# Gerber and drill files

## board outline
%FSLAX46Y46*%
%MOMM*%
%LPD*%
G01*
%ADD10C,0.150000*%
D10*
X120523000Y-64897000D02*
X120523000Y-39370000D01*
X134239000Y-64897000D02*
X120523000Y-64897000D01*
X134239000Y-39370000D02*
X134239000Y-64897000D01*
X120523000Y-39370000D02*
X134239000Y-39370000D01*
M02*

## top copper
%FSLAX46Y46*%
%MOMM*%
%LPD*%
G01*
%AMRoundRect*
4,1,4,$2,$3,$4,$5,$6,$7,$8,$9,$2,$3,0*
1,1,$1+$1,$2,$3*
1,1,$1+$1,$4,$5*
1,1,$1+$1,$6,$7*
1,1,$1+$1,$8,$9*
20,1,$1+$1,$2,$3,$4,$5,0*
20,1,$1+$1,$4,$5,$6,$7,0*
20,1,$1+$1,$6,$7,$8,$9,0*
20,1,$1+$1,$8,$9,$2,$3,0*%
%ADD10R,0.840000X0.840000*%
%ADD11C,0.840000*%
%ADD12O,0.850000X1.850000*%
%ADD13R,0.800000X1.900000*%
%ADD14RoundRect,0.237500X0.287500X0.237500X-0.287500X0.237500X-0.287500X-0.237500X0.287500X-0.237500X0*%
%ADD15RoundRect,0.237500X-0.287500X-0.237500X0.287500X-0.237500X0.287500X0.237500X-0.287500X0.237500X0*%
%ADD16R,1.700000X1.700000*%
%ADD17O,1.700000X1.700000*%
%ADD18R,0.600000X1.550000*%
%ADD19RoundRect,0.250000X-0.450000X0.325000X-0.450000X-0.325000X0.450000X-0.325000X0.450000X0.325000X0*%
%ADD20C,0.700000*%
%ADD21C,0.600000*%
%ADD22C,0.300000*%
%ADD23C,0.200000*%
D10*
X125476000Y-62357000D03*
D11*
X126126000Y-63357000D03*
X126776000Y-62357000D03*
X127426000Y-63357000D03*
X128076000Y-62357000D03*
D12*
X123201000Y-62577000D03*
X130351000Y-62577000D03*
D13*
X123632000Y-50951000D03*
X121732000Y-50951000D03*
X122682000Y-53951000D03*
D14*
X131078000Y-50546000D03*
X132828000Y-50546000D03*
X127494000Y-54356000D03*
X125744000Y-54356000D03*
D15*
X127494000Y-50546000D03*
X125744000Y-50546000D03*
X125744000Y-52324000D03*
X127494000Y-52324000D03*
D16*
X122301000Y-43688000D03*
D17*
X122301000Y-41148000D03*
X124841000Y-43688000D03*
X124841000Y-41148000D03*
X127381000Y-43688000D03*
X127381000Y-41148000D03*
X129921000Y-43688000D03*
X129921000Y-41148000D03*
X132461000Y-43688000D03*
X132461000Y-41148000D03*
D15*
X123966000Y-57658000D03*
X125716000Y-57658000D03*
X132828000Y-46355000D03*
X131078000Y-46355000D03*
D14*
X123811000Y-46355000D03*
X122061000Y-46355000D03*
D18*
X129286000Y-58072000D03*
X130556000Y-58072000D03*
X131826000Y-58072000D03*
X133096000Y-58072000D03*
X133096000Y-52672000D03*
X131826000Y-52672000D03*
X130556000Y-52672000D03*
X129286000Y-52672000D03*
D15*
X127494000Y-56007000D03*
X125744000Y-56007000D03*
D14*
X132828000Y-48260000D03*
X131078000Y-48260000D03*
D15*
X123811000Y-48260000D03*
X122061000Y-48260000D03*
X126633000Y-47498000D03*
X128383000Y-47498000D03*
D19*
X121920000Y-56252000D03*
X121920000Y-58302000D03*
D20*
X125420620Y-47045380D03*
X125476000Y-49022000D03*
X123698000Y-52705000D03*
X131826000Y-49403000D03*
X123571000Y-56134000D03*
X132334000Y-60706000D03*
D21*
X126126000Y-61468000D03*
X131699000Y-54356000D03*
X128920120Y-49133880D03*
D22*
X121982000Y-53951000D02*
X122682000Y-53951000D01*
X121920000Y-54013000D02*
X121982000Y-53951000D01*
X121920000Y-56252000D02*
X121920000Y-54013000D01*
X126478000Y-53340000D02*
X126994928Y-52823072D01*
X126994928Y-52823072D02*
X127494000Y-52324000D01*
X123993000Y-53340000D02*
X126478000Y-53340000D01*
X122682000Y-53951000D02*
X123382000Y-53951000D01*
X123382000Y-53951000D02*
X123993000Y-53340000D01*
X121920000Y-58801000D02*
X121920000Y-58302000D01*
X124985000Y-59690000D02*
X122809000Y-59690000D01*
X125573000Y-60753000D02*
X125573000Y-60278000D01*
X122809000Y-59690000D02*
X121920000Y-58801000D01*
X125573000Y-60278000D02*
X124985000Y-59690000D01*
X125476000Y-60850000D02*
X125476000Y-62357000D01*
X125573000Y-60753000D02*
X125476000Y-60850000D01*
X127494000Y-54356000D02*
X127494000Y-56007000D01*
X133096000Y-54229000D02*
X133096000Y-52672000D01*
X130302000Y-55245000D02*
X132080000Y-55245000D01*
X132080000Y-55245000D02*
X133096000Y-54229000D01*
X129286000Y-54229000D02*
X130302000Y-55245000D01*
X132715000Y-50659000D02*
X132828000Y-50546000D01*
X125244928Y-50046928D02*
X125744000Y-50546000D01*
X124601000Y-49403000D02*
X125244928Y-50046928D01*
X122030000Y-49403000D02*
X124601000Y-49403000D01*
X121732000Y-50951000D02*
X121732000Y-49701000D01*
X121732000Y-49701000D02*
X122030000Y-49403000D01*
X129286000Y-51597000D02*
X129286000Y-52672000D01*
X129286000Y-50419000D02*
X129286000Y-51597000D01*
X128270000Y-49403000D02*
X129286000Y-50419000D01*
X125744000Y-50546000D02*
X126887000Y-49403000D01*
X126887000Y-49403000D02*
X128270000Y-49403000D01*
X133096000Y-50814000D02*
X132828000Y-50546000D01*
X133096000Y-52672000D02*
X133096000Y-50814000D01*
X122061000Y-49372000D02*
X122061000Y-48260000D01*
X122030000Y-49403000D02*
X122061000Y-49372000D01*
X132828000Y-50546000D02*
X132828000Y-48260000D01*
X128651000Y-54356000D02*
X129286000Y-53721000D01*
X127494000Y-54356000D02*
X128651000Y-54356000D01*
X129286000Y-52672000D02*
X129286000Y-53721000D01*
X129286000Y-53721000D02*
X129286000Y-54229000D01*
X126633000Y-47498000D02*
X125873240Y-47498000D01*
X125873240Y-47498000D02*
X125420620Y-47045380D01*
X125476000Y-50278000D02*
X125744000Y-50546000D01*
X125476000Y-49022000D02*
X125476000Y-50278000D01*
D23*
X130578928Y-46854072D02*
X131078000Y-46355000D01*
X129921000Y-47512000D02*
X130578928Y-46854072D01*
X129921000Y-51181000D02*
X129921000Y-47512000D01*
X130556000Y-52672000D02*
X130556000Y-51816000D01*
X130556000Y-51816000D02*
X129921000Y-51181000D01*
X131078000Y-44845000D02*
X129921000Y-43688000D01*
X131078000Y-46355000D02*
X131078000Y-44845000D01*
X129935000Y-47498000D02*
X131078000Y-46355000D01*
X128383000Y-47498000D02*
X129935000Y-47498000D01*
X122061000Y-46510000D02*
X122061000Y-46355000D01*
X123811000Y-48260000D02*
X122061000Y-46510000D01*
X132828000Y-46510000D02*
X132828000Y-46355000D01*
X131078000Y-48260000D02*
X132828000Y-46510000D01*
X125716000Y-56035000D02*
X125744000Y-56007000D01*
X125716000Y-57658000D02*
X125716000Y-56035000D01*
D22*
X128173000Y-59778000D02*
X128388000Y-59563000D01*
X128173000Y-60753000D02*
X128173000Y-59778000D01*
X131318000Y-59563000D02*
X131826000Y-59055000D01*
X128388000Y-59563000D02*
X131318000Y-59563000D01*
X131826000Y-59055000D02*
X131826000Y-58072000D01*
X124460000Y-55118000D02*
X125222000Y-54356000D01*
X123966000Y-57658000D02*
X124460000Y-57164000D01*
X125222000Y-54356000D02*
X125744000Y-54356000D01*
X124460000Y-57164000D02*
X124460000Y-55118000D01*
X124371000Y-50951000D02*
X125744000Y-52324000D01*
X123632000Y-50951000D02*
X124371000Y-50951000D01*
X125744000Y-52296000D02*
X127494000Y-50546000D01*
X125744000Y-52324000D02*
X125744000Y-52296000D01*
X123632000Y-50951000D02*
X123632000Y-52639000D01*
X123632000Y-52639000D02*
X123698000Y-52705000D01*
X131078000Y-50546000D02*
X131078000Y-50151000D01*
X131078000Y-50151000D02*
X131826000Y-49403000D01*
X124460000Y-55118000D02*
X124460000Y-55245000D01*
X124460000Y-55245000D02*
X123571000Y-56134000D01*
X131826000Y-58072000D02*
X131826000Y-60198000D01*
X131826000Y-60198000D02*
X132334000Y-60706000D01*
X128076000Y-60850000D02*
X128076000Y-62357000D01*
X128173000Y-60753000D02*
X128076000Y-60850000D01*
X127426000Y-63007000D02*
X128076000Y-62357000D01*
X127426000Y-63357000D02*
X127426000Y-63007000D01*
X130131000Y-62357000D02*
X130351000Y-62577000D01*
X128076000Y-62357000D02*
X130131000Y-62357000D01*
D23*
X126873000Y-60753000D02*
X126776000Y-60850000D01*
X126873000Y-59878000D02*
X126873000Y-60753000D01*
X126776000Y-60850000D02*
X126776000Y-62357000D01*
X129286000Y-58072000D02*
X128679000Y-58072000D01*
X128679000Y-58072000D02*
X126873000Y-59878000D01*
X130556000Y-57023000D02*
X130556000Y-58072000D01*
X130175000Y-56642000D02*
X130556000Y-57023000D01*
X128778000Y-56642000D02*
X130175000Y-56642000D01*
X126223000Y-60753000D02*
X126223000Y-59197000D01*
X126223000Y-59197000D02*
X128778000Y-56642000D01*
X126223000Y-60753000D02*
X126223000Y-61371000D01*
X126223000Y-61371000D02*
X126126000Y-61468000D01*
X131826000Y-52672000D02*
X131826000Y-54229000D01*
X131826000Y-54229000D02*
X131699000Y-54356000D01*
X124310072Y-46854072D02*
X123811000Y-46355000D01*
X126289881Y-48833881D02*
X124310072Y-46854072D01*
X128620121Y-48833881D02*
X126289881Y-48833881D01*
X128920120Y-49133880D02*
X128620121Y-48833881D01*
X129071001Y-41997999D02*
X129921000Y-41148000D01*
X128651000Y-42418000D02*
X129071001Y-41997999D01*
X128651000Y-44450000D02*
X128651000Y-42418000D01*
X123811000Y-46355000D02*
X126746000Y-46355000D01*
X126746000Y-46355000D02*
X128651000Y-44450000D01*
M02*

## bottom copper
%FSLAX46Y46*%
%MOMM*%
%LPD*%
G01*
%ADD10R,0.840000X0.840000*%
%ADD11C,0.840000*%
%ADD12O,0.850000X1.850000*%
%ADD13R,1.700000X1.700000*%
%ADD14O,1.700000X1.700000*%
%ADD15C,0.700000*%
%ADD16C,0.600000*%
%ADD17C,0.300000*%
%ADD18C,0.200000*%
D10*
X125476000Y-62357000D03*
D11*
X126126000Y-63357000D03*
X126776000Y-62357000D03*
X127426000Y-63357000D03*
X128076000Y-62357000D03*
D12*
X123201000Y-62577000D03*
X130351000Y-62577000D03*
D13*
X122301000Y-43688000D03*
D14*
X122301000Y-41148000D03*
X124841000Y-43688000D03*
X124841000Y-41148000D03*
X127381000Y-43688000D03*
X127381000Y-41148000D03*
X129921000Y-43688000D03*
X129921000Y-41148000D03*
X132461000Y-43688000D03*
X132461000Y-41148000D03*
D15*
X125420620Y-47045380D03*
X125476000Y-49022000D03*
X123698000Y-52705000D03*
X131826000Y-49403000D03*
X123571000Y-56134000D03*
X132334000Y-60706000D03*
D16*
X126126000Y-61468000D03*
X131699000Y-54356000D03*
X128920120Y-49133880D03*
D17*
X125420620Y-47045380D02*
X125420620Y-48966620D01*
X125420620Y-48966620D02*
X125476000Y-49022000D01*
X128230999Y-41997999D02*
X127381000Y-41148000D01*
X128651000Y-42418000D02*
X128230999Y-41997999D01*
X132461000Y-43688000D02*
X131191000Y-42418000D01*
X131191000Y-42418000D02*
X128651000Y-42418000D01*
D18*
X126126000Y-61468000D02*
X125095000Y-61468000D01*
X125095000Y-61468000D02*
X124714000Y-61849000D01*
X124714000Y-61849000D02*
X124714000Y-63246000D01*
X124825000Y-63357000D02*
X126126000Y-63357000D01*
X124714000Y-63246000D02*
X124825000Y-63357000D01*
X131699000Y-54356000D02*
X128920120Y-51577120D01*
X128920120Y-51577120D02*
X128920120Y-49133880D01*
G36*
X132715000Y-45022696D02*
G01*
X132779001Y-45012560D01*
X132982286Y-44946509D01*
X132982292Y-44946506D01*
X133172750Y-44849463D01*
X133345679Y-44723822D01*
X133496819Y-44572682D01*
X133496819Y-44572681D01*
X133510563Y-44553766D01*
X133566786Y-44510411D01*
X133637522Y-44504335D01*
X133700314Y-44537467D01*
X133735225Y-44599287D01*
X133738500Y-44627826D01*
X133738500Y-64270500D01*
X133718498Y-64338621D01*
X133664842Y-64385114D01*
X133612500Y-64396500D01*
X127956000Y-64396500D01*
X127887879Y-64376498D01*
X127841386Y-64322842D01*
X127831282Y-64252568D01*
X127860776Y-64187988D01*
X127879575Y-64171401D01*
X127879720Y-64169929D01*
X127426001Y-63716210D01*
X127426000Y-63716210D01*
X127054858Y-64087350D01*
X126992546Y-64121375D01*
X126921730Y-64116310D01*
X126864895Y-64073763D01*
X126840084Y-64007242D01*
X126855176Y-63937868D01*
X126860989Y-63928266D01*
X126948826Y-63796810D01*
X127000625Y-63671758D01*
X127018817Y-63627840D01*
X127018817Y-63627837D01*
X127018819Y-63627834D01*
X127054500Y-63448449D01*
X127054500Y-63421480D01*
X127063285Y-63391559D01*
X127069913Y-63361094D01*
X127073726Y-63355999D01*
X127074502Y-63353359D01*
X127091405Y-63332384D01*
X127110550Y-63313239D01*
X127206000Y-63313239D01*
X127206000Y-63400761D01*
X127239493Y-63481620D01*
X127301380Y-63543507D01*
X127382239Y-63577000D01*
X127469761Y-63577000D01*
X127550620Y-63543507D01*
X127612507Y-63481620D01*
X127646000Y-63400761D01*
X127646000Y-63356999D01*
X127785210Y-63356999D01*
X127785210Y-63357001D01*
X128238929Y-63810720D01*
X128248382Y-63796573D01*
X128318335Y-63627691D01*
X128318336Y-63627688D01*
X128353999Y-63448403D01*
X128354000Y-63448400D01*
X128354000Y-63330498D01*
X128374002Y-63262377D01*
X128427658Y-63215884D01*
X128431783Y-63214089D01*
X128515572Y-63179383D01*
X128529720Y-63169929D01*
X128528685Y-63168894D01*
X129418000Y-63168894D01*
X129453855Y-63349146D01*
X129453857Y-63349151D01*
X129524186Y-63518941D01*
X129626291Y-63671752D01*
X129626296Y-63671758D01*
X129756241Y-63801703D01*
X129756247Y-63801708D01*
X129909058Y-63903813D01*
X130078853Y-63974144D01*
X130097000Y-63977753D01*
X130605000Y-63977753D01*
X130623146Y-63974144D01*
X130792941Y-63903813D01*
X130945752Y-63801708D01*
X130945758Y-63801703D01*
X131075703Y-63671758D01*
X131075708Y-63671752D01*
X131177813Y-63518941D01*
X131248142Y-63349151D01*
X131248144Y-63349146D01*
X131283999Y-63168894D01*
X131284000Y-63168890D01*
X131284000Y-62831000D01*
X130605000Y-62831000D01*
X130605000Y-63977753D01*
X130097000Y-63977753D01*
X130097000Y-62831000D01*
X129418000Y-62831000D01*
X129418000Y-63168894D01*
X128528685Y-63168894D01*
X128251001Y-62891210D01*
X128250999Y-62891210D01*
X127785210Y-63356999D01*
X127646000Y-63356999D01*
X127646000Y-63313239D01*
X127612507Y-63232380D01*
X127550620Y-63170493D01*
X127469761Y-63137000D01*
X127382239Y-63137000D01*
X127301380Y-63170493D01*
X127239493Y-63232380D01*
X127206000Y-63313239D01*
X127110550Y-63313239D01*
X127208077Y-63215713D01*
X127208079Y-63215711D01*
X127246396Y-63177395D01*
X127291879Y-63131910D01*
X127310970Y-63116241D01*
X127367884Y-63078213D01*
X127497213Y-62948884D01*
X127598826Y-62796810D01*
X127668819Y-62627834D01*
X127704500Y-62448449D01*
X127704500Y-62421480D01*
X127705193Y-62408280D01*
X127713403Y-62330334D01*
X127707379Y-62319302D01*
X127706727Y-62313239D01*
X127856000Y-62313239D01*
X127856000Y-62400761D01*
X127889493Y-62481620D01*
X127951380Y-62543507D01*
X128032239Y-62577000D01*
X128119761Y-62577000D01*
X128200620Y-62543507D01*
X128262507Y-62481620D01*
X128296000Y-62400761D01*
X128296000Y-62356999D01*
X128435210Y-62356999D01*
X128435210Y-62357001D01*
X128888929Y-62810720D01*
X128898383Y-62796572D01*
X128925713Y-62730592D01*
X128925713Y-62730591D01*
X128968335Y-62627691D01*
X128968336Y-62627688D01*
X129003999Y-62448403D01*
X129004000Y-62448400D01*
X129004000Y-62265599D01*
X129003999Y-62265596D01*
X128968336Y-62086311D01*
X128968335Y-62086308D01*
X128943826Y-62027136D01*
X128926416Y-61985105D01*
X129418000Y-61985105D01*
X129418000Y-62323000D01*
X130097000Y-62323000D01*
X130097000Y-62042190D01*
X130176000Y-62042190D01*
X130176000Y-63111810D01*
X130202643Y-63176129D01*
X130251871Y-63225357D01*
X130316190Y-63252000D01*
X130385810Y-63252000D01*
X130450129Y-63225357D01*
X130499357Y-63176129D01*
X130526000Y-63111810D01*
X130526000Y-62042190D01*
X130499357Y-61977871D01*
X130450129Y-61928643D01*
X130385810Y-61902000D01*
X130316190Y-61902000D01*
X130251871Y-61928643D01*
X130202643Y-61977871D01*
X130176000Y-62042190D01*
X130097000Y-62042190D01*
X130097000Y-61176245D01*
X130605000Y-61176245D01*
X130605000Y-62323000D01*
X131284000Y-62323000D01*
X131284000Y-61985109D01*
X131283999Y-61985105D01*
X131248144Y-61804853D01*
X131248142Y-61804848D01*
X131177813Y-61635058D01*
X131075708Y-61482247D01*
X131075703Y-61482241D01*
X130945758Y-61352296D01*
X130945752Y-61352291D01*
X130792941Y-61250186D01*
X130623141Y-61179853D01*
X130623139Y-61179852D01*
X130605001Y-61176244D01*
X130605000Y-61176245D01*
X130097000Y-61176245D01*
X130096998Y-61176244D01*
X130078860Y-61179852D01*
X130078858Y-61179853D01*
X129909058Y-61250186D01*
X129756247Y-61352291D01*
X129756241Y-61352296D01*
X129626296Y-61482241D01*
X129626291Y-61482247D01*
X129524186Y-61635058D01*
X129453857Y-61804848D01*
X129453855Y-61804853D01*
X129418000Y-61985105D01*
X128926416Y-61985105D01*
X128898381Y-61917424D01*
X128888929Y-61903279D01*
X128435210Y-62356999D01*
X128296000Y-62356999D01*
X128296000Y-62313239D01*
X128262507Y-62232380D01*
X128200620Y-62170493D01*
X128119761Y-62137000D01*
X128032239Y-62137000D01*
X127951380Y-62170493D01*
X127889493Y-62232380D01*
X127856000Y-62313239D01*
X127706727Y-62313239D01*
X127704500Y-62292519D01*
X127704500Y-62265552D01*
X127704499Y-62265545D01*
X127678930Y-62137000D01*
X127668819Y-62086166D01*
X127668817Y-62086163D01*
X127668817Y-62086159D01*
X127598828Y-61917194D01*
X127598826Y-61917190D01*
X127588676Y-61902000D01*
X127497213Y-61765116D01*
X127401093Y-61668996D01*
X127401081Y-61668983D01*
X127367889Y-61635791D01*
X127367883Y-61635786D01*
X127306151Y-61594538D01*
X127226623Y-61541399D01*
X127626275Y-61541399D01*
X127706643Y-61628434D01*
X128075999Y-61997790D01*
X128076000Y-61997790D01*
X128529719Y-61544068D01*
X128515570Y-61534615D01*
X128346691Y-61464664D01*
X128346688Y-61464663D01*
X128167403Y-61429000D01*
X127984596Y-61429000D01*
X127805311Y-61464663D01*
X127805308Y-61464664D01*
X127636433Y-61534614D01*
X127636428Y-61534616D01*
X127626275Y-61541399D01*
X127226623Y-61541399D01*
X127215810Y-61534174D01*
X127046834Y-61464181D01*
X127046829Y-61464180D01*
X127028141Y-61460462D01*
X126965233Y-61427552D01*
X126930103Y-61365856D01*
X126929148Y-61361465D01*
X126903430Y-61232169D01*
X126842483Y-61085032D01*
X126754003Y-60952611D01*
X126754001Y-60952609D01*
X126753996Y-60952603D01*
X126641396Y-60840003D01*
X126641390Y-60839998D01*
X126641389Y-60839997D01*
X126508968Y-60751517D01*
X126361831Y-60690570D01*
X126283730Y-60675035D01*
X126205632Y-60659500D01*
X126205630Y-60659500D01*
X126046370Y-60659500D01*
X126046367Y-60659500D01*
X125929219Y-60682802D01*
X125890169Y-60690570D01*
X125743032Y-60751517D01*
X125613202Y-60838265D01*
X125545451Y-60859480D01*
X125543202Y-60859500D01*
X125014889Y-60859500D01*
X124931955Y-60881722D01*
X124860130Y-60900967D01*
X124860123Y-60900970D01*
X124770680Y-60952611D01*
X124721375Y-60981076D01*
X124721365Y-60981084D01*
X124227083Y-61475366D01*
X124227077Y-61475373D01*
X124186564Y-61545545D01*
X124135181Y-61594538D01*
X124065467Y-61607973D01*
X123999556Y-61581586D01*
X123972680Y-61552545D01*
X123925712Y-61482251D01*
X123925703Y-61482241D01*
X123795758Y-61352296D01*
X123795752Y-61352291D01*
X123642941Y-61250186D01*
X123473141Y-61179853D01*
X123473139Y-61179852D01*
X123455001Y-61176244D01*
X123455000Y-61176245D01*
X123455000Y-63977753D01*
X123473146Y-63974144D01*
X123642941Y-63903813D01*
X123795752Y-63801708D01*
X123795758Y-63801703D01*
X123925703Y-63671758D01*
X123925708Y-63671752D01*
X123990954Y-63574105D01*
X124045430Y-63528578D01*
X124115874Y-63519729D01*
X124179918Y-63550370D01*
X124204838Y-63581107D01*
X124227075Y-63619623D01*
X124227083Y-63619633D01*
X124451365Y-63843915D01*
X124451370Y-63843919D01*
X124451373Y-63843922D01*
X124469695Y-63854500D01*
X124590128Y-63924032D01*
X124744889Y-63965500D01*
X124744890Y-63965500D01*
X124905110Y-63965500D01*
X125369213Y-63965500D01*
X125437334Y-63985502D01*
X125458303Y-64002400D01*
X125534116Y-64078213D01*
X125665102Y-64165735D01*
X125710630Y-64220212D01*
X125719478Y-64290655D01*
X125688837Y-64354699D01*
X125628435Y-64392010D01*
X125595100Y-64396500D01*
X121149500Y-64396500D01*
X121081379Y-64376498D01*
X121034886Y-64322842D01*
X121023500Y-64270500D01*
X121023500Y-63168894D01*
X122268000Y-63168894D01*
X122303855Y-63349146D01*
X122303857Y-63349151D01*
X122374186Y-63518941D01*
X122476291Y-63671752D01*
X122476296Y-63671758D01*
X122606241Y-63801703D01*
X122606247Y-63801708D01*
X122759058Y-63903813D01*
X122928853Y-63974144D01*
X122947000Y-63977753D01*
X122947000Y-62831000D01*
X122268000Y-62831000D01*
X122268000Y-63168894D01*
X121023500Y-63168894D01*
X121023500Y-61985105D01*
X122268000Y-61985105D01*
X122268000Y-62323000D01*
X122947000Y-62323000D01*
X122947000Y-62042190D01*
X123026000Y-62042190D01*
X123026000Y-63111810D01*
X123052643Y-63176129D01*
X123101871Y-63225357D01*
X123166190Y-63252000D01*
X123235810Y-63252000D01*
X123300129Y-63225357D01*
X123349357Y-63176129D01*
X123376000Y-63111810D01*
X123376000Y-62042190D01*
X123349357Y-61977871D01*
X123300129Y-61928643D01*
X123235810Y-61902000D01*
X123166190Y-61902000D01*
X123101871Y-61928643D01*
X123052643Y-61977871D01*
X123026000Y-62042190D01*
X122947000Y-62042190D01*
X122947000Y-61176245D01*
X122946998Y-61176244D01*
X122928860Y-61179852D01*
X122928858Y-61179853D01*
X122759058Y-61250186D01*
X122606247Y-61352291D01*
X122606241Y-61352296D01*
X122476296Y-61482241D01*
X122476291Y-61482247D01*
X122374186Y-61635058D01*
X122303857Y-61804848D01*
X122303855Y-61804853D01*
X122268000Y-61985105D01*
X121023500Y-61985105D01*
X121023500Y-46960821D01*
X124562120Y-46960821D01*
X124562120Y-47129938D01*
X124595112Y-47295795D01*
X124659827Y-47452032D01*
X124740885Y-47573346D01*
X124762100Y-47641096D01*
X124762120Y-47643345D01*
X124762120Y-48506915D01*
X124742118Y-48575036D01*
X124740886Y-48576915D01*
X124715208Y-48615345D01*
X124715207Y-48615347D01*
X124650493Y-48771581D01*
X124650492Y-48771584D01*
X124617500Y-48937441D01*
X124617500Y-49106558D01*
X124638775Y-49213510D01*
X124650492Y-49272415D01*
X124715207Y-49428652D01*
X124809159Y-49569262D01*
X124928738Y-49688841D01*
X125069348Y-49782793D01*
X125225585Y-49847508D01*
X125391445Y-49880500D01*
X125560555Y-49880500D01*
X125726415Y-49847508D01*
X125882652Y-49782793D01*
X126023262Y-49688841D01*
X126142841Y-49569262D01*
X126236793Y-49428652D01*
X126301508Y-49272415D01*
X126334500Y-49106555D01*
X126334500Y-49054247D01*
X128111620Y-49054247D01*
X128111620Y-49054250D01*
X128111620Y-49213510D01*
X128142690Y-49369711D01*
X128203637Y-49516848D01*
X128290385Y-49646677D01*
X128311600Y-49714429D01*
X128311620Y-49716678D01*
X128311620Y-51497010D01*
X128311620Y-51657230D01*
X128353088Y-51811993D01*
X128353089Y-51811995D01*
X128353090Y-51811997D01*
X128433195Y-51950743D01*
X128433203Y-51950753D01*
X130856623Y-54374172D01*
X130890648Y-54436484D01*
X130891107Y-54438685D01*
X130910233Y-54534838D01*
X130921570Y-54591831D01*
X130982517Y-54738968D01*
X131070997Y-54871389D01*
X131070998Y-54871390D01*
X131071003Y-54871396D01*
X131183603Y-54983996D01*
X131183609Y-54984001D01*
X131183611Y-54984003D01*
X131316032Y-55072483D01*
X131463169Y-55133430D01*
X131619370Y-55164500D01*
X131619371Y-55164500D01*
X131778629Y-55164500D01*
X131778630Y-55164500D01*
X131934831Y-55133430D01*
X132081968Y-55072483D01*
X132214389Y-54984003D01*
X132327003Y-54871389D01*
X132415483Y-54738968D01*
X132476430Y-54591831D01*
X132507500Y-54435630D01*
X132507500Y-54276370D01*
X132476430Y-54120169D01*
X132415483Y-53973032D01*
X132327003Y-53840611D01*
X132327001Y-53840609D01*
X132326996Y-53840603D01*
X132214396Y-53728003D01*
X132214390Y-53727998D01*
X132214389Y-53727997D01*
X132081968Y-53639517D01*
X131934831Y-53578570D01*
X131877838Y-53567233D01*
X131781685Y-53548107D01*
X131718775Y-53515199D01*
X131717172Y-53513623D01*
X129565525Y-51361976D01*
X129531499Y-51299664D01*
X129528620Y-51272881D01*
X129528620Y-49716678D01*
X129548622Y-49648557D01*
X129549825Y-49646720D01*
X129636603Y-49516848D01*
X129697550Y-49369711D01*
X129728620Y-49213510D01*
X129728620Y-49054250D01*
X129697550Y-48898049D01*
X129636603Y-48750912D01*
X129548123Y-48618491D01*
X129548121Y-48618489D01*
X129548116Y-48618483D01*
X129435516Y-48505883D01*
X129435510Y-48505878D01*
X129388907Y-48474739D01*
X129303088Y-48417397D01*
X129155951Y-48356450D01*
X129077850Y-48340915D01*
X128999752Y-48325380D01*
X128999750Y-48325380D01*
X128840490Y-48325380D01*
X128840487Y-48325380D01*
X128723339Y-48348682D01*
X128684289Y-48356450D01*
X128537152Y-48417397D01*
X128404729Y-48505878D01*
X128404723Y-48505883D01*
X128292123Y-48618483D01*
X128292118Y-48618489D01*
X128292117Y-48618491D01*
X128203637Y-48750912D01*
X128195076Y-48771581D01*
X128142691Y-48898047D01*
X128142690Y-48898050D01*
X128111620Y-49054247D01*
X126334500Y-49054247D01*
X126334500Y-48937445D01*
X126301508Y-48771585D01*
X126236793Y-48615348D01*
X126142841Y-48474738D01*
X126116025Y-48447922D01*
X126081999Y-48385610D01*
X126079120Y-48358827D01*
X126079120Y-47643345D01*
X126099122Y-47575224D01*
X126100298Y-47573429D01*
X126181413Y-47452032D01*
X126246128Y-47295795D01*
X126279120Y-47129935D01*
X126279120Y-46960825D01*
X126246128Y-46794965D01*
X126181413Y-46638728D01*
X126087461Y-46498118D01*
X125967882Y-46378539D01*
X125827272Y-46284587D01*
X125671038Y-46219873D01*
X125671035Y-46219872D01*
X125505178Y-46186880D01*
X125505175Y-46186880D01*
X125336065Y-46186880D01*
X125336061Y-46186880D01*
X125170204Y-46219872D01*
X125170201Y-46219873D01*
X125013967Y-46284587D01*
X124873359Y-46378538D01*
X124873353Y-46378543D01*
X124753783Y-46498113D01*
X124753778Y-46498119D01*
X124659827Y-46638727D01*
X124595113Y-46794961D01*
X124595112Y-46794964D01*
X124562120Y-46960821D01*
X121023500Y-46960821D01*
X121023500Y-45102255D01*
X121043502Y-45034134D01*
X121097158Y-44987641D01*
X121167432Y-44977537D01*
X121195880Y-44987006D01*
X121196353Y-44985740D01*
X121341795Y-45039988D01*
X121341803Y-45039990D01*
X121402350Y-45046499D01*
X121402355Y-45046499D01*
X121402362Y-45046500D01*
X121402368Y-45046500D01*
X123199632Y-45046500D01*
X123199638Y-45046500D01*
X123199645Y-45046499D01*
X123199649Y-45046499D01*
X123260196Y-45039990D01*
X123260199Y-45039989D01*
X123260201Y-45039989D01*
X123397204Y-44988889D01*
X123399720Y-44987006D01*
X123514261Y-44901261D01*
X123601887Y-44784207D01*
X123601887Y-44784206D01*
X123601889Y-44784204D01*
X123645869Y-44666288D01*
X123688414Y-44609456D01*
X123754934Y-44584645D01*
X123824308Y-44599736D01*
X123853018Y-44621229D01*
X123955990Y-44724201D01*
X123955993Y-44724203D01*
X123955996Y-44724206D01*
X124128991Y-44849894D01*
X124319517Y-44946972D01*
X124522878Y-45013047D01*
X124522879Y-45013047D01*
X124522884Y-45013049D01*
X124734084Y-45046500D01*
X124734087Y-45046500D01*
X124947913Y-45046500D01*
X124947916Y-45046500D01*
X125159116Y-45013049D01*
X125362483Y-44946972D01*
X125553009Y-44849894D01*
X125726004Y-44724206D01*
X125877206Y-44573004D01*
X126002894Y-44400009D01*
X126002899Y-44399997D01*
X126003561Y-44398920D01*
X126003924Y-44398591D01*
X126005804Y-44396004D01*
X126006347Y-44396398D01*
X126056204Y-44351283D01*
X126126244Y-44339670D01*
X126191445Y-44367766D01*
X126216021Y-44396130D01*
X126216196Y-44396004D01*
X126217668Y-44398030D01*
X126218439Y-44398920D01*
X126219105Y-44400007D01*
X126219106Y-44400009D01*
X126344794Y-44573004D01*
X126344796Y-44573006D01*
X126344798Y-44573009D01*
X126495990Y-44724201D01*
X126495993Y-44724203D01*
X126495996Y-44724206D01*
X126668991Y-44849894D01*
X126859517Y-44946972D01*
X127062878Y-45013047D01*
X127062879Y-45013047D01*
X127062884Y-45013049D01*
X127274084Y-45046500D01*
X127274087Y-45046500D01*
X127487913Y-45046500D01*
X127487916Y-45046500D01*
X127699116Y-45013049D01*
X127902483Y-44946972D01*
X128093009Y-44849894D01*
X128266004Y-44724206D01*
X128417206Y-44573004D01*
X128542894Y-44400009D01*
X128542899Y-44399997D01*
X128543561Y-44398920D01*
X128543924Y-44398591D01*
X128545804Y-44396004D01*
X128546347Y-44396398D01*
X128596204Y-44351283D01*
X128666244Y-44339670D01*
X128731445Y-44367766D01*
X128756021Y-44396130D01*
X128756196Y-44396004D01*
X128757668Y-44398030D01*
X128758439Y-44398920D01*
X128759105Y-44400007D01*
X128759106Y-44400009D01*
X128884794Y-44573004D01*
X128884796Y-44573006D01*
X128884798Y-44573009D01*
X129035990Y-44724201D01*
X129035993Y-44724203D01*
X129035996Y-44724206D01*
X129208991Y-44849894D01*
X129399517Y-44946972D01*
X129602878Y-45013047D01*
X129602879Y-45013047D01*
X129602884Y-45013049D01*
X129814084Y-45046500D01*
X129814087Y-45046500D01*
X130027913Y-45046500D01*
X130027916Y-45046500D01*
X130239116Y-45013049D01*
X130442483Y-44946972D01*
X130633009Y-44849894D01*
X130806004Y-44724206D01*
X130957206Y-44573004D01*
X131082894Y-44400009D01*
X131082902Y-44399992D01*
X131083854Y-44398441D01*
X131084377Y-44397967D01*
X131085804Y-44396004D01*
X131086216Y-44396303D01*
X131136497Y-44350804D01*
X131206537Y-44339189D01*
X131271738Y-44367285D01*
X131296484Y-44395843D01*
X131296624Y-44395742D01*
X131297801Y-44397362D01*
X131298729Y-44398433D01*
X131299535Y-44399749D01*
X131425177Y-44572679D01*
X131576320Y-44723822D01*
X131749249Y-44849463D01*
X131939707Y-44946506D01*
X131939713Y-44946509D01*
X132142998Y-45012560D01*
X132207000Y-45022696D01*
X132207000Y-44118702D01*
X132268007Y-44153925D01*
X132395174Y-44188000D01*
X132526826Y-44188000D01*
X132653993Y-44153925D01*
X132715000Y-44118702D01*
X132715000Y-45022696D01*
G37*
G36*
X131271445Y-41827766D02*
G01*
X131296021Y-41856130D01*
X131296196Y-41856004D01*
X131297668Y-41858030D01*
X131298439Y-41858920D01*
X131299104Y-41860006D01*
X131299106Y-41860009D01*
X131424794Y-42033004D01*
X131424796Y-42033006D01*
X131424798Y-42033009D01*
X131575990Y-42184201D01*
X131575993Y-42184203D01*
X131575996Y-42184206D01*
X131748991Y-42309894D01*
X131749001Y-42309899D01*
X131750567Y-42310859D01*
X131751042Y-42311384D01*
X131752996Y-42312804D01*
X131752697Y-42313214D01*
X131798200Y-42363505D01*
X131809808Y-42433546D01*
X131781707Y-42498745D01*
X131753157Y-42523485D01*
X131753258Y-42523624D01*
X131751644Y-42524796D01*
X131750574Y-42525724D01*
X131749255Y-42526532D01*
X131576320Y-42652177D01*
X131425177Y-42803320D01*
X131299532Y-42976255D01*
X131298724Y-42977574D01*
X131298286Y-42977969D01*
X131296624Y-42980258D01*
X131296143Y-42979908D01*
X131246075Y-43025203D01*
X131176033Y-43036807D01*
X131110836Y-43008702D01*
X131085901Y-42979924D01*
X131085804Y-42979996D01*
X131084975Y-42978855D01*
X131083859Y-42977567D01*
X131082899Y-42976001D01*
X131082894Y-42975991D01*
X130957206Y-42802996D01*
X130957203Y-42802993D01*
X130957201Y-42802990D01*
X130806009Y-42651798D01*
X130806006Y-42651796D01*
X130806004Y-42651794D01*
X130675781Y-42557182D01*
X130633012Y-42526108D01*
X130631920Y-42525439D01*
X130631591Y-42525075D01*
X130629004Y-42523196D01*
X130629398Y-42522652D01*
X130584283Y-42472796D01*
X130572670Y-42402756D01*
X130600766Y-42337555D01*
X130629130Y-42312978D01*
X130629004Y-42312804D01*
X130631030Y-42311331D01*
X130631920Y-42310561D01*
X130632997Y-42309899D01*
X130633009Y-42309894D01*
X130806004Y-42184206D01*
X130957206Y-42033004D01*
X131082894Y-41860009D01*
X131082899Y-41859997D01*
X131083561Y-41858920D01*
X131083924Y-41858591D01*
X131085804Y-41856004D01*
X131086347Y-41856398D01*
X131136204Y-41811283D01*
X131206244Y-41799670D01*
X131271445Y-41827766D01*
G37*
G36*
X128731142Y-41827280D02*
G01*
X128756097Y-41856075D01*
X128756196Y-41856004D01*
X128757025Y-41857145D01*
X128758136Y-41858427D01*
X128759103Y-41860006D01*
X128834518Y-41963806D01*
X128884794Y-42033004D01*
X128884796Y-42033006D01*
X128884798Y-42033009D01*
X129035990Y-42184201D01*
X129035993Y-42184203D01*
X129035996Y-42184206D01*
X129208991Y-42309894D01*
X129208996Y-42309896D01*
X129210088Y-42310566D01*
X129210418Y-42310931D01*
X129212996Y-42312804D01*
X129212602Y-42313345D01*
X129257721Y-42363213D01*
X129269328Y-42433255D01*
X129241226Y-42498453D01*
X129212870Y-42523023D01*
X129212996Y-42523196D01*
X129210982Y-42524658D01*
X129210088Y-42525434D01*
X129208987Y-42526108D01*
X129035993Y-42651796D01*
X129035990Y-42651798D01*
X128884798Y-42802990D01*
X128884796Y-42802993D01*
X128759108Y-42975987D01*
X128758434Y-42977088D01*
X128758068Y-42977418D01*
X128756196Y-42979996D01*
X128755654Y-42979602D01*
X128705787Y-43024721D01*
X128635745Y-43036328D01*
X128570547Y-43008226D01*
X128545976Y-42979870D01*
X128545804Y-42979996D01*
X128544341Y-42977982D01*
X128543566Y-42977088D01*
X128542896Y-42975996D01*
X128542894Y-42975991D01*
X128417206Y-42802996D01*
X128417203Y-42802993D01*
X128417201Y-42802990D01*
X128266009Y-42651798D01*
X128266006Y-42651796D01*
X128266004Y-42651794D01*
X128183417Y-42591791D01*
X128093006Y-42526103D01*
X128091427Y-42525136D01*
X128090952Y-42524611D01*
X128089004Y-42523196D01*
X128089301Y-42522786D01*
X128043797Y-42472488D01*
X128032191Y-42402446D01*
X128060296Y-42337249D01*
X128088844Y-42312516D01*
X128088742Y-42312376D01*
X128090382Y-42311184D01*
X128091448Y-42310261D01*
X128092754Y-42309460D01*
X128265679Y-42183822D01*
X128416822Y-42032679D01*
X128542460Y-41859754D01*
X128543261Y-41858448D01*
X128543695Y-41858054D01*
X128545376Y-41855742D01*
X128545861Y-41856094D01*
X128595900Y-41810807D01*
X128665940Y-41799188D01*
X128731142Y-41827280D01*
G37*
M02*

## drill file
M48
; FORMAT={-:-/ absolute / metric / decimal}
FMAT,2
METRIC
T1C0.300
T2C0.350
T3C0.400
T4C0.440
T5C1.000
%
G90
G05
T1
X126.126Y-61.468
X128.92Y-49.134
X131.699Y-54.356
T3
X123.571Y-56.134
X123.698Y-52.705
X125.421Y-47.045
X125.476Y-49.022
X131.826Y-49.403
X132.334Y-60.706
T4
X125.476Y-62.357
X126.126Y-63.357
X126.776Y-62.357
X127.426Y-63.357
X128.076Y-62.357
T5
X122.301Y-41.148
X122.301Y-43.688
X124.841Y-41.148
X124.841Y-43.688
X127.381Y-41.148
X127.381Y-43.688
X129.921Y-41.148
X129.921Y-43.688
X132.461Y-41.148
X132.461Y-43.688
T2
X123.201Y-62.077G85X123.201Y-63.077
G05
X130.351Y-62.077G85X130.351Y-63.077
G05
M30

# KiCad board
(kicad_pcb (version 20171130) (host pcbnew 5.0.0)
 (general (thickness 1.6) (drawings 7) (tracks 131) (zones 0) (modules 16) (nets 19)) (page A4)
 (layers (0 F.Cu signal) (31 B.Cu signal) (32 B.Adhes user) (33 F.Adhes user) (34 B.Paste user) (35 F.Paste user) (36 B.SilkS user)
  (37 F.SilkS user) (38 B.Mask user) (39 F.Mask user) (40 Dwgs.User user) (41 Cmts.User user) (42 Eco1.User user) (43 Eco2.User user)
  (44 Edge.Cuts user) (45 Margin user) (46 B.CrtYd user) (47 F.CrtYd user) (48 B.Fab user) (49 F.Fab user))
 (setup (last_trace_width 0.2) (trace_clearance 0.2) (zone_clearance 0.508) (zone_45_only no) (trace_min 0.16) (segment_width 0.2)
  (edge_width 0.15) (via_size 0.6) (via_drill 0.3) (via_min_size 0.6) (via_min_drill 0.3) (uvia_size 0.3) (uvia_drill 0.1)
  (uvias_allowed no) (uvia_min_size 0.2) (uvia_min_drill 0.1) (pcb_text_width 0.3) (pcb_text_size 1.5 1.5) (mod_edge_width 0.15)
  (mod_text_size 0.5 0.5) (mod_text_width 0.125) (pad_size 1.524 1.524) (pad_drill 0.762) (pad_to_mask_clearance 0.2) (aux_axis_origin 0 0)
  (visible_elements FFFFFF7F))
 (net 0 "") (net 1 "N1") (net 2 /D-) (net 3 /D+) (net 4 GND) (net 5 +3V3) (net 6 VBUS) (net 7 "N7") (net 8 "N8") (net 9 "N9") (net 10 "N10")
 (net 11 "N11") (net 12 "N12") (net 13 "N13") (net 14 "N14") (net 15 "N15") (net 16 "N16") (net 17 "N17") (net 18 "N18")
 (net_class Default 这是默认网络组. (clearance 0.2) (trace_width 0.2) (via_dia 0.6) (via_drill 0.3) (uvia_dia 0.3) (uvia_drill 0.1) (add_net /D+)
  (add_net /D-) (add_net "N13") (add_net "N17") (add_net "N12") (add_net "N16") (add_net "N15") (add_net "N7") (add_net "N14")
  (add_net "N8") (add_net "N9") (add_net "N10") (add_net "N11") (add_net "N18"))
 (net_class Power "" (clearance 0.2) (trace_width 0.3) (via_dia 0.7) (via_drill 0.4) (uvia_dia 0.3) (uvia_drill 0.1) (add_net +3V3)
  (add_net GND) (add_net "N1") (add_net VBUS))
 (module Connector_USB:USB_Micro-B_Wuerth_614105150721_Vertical (layer F.Cu) (at 125.476 62.357)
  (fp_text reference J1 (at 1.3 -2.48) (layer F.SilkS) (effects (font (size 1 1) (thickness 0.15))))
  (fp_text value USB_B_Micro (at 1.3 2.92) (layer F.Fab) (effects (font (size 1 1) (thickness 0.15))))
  (pad 1 thru_hole rect (at 0 0) (size 0.84 0.84) (drill 0.44) (layers *.Cu *.Mask) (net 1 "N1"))
  (pad 2 thru_hole circle (at 0.65 1) (size 0.84 0.84) (drill 0.44) (layers *.Cu *.Mask) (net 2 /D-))
  (pad 3 thru_hole circle (at 1.3 0) (size 0.84 0.84) (drill 0.44) (layers *.Cu *.Mask) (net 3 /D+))
  (pad 4 thru_hole circle (at 1.95 1) (size 0.84 0.84) (drill 0.44) (layers *.Cu *.Mask) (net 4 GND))
  (pad 5 thru_hole circle (at 2.6 0) (size 0.84 0.84) (drill 0.44) (layers *.Cu *.Mask) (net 4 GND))
  (pad 6 thru_hole oval (at -2.275 0.22) (size 0.85 1.85) (drill oval 0.35 1.35) (layers *.Cu *.Mask) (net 4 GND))
  (pad 6 thru_hole oval (at 4.875 0.22) (size 0.85 1.85) (drill oval 0.35 1.35) (layers *.Cu *.Mask) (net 4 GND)))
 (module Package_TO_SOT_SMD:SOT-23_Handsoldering (layer F.Cu) (at 122.682 52.451 270)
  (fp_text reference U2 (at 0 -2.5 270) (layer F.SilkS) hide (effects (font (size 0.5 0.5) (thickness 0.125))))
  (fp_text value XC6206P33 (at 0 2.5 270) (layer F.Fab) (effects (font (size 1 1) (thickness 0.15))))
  (pad 1 smd rect (at -1.5 -0.95 270) (size 1.9 0.8) (layers F.Cu F.Paste F.Mask) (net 4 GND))
  (pad 2 smd rect (at -1.5 0.95 270) (size 1.9 0.8) (layers F.Cu F.Paste F.Mask) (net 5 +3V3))
  (pad 3 smd rect (at 1.5 0 270) (size 1.9 0.8) (layers F.Cu F.Paste F.Mask) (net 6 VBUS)))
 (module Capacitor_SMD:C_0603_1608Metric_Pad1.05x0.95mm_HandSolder (layer F.Cu) (at 131.953 50.546 180)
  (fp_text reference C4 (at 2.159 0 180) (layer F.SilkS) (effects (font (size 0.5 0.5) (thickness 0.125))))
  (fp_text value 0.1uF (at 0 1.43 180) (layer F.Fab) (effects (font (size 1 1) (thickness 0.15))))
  (pad 2 smd roundrect (at 0.875 0 180) (size 1.05 0.95) (layers F.Cu F.Paste F.Mask) (roundrect_rratio 0.25) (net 4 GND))
  (pad 1 smd roundrect (at -0.875 0 180) (size 1.05 0.95) (layers F.Cu F.Paste F.Mask) (roundrect_rratio 0.25) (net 5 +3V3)))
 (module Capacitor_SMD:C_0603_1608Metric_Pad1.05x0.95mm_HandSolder (layer F.Cu) (at 126.619 54.356 180)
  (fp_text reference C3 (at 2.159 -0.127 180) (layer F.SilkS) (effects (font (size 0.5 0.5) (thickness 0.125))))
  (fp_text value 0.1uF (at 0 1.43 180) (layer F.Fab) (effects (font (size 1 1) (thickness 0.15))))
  (pad 1 smd roundrect (at -0.875 0 180) (size 1.05 0.95) (layers F.Cu F.Paste F.Mask) (roundrect_rratio 0.25) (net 5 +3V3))
  (pad 2 smd roundrect (at 0.875 0 180) (size 1.05 0.95) (layers F.Cu F.Paste F.Mask) (roundrect_rratio 0.25) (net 4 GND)))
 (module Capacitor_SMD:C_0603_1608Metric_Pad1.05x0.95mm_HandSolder (layer F.Cu) (at 126.619 50.546)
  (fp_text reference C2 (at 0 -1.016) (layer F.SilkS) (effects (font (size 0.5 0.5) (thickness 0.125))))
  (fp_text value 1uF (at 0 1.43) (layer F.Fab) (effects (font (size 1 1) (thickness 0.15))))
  (pad 2 smd roundrect (at 0.875 0) (size 1.05 0.95) (layers F.Cu F.Paste F.Mask) (roundrect_rratio 0.25) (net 4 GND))
  (pad 1 smd roundrect (at -0.875 0) (size 1.05 0.95) (layers F.Cu F.Paste F.Mask) (roundrect_rratio 0.25) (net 5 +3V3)))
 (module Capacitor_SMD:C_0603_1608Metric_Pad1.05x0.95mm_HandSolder (layer F.Cu) (at 126.619 52.324)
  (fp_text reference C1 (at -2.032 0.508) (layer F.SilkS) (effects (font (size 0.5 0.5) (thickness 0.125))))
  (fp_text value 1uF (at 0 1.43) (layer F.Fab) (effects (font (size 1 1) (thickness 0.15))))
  (pad 1 smd roundrect (at -0.875 0) (size 1.05 0.95) (layers F.Cu F.Paste F.Mask) (roundrect_rratio 0.25) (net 4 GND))
  (pad 2 smd roundrect (at 0.875 0) (size 1.05 0.95) (layers F.Cu F.Paste F.Mask) (roundrect_rratio 0.25) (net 6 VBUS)))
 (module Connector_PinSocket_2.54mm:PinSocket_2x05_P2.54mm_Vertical (layer B.Cu) (at 122.301 43.688 270)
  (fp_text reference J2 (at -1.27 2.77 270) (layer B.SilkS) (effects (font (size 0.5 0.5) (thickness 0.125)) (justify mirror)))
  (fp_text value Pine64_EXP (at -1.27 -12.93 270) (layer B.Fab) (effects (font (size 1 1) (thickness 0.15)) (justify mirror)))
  (pad 1 thru_hole rect (at 0 0 270) (size 1.7 1.7) (drill 1) (layers *.Cu *.Mask) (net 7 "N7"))
  (pad 2 thru_hole oval (at -2.54 0 270) (size 1.7 1.7) (drill 1) (layers *.Cu *.Mask) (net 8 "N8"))
  (pad 3 thru_hole oval (at 0 -2.54 270) (size 1.7 1.7) (drill 1) (layers *.Cu *.Mask) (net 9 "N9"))
  (pad 4 thru_hole oval (at -2.54 -2.54 270) (size 1.7 1.7) (drill 1) (layers *.Cu *.Mask) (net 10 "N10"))
  (pad 5 thru_hole oval (at 0 -5.08 270) (size 1.7 1.7) (drill 1) (layers *.Cu *.Mask) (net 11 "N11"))
  (pad 6 thru_hole oval (at -2.54 -5.08 270) (size 1.7 1.7) (drill 1) (layers *.Cu *.Mask) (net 4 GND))
  (pad 7 thru_hole oval (at 0 -7.62 270) (size 1.7 1.7) (drill 1) (layers *.Cu *.Mask) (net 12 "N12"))
  (pad 8 thru_hole oval (at -2.54 -7.62 270) (size 1.7 1.7) (drill 1) (layers *.Cu *.Mask) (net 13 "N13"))
  (pad 9 thru_hole oval (at 0 -10.16 270) (size 1.7 1.7) (drill 1) (layers *.Cu *.Mask) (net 4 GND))
  (pad 10 thru_hole oval (at -2.54 -10.16 270) (size 1.7 1.7) (drill 1) (layers *.Cu *.Mask) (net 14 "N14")))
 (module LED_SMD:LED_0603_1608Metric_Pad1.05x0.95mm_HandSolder (layer F.Cu) (at 124.841 57.658)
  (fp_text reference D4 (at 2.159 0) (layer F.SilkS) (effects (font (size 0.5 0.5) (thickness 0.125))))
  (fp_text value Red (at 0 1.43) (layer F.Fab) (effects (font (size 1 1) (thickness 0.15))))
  (pad 1 smd roundrect (at -0.875 0) (size 1.05 0.95) (layers F.Cu F.Paste F.Mask) (roundrect_rratio 0.25) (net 4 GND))
  (pad 2 smd roundrect (at 0.875 0) (size 1.05 0.95) (layers F.Cu F.Paste F.Mask) (roundrect_rratio 0.25) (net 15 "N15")))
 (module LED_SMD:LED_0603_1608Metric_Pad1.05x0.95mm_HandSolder (layer F.Cu) (at 131.953 46.355)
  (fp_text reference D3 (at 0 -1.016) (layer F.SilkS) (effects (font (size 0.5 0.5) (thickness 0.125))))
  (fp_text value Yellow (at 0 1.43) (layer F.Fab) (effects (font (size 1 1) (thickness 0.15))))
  (pad 2 smd roundrect (at 0.875 0) (size 1.05 0.95) (layers F.Cu F.Paste F.Mask) (roundrect_rratio 0.25) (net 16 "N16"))
  (pad 1 smd roundrect (at -0.875 0) (size 1.05 0.95) (layers F.Cu F.Paste F.Mask) (roundrect_rratio 0.25) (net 12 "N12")))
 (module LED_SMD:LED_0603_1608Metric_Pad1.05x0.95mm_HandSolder (layer F.Cu) (at 122.936 46.355 180)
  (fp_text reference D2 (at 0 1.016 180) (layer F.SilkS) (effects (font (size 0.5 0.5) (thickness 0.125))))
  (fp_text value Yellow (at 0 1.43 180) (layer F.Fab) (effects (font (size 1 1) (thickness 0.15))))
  (pad 1 smd roundrect (at -0.875 0 180) (size 1.05 0.95) (layers F.Cu F.Paste F.Mask) (roundrect_rratio 0.25) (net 13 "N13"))
  (pad 2 smd roundrect (at 0.875 0 180) (size 1.05 0.95) (layers F.Cu F.Paste F.Mask) (roundrect_rratio 0.25) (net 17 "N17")))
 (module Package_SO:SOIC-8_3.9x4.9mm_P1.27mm (layer F.Cu) (at 131.191 55.372 90)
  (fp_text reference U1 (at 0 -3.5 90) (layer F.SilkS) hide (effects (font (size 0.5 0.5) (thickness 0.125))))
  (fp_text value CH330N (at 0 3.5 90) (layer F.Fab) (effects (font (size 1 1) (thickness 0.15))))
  (pad 1 smd rect (at -2.7 -1.905 90) (size 1.55 0.6) (layers F.Cu F.Paste F.Mask) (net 3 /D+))
  (pad 2 smd rect (at -2.7 -0.635 90) (size 1.55 0.6) (layers F.Cu F.Paste F.Mask) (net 2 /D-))
  (pad 3 smd rect (at -2.7 0.635 90) (size 1.55 0.6) (layers F.Cu F.Paste F.Mask) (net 4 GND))
  (pad 4 smd rect (at -2.7 1.905 90) (size 1.55 0.6) (layers F.Cu F.Paste F.Mask) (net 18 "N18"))
  (pad 5 smd rect (at 2.7 1.905 90) (size 1.55 0.6) (layers F.Cu F.Paste F.Mask) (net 5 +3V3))
  (pad 6 smd rect (at 2.7 0.635 90) (size 1.55 0.6) (layers F.Cu F.Paste F.Mask) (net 13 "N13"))
  (pad 7 smd rect (at 2.7 -0.635 90) (size 1.55 0.6) (layers F.Cu F.Paste F.Mask) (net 12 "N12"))
  (pad 8 smd rect (at 2.7 -1.905 90) (size 1.55 0.6) (layers F.Cu F.Paste F.Mask) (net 5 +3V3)))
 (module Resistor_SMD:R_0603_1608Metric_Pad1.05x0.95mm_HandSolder (layer F.Cu) (at 126.619 56.007)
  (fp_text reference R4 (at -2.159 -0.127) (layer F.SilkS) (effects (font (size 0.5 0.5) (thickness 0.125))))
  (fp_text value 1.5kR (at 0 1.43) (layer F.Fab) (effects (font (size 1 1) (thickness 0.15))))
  (pad 2 smd roundrect (at 0.875 0) (size 1.05 0.95) (layers F.Cu F.Paste F.Mask) (roundrect_rratio 0.25) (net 5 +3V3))
  (pad 1 smd roundrect (at -0.875 0) (size 1.05 0.95) (layers F.Cu F.Paste F.Mask) (roundrect_rratio 0.25) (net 15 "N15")))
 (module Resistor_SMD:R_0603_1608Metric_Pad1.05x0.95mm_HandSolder (layer F.Cu) (at 131.953 48.26 180)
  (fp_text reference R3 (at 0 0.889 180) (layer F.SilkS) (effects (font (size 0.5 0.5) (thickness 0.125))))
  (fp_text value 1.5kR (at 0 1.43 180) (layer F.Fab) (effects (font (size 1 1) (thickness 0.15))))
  (pad 1 smd roundrect (at -0.875 0 180) (size 1.05 0.95) (layers F.Cu F.Paste F.Mask) (roundrect_rratio 0.25) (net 5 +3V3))
  (pad 2 smd roundrect (at 0.875 0 180) (size 1.05 0.95) (layers F.Cu F.Paste F.Mask) (roundrect_rratio 0.25) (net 16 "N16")))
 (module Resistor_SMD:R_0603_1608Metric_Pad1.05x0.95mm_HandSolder (layer F.Cu) (at 122.936 48.26)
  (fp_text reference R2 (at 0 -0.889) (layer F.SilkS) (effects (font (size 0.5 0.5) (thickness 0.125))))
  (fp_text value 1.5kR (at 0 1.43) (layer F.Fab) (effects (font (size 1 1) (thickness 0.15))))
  (pad 2 smd roundrect (at 0.875 0) (size 1.05 0.95) (layers F.Cu F.Paste F.Mask) (roundrect_rratio 0.25) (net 17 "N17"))
  (pad 1 smd roundrect (at -0.875 0) (size 1.05 0.95) (layers F.Cu F.Paste F.Mask) (roundrect_rratio 0.25) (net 5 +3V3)))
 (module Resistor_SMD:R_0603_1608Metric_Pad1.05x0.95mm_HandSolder (layer F.Cu) (at 127.508 47.498)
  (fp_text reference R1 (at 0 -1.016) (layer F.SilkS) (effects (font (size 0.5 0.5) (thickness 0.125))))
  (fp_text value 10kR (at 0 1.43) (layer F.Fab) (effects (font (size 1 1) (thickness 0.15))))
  (pad 1 smd roundrect (at -0.875 0) (size 1.05 0.95) (layers F.Cu F.Paste F.Mask) (roundrect_rratio 0.25) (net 5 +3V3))
  (pad 2 smd roundrect (at 0.875 0) (size 1.05 0.95) (layers F.Cu F.Paste F.Mask) (roundrect_rratio 0.25) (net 12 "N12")))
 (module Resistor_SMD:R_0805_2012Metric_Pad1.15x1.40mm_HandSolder (layer F.Cu) (at 121.92 57.277 270)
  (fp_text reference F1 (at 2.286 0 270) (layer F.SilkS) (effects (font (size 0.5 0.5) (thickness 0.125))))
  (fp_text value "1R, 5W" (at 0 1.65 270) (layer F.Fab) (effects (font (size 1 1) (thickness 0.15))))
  (pad 1 smd roundrect (at -1.025 0 270) (size 1.15 1.4) (layers F.Cu F.Paste F.Mask) (roundrect_rratio 0.217391) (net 6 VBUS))
  (pad 2 smd roundrect (at 1.025 0 270) (size 1.15 1.4) (layers F.Cu F.Paste F.Mask) (roundrect_rratio 0.217391) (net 1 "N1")))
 (gr_line (start 120.523 64.897) (end 120.523 39.37) (layer Edge.Cuts) (width 0.15))
 (gr_line (start 134.239 64.897) (end 120.523 64.897) (layer Edge.Cuts) (width 0.15))
 (gr_line (start 134.239 39.37) (end 134.239 64.897) (layer Edge.Cuts) (width 0.15))
 (gr_line (start 120.523 39.37) (end 134.239 39.37) (layer Edge.Cuts) (width 0.15))
 (segment (start 121.982 53.951) (end 122.682 53.951) (width 0.3) (layer F.Cu) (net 6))
 (segment (start 121.92 54.013) (end 121.982 53.951) (width 0.3) (layer F.Cu) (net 6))
 (segment (start 121.92 56.252) (end 121.92 54.013) (width 0.3) (layer F.Cu) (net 6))
 (segment (start 126.478 53.34) (end 126.994928 52.823072) (width 0.3) (layer F.Cu) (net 6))
 (segment (start 126.994928 52.823072) (end 127.494 52.324) (width 0.3) (layer F.Cu) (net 6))
 (segment (start 123.993 53.34) (end 126.478 53.34) (width 0.3) (layer F.Cu) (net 6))
 (segment (start 122.682 53.951) (end 123.382 53.951) (width 0.3) (layer F.Cu) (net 6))
 (segment (start 123.382 53.951) (end 123.993 53.34) (width 0.3) (layer F.Cu) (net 6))
 (segment (start 121.92 58.801) (end 121.92 58.302) (width 0.3) (layer F.Cu) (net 1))
 (segment (start 124.985 59.69) (end 122.809 59.69) (width 0.3) (layer F.Cu) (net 1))
 (segment (start 125.573 60.753) (end 125.573 60.278) (width 0.3) (layer F.Cu) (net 1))
 (segment (start 122.809 59.69) (end 121.92 58.801) (width 0.3) (layer F.Cu) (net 1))
 (segment (start 125.573 60.278) (end 124.985 59.69) (width 0.3) (layer F.Cu) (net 1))
 (segment (start 125.476 60.85) (end 125.476 62.357) (width 0.3) (layer F.Cu) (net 1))
 (segment (start 125.573 60.753) (end 125.476 60.85) (width 0.3) (layer F.Cu) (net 1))
 (segment (start 127.494 54.356) (end 127.494 56.007) (width 0.3) (layer F.Cu) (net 5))
 (segment (start 133.096 54.229) (end 133.096 52.672) (width 0.3) (layer F.Cu) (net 5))
 (segment (start 130.302 55.245) (end 132.08 55.245) (width 0.3) (layer F.Cu) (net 5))
 (segment (start 132.08 55.245) (end 133.096 54.229) (width 0.3) (layer F.Cu) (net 5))
 (segment (start 129.286 54.229) (end 130.302 55.245) (width 0.3) (layer F.Cu) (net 5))
 (segment (start 132.715 50.659) (end 132.828 50.546) (width 0.3) (layer F.Cu) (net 5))
 (segment (start 125.244928 50.046928) (end 125.744 50.546) (width 0.3) (layer F.Cu) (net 5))
 (segment (start 124.601 49.403) (end 125.244928 50.046928) (width 0.3) (layer F.Cu) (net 5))
 (segment (start 122.03 49.403) (end 124.601 49.403) (width 0.3) (layer F.Cu) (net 5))
 (segment (start 121.732 50.951) (end 121.732 49.701) (width 0.3) (layer F.Cu) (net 5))
 (segment (start 121.732 49.701) (end 122.03 49.403) (width 0.3) (layer F.Cu) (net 5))
 (segment (start 129.286 51.597) (end 129.286 52.672) (width 0.3) (layer F.Cu) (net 5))
 (segment (start 129.286 50.419) (end 129.286 51.597) (width 0.3) (layer F.Cu) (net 5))
 (segment (start 128.27 49.403) (end 129.286 50.419) (width 0.3) (layer F.Cu) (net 5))
 (segment (start 125.744 50.546) (end 126.887 49.403) (width 0.3) (layer F.Cu) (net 5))
 (segment (start 126.887 49.403) (end 128.27 49.403) (width 0.3) (layer F.Cu) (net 5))
 (segment (start 133.096 50.814) (end 132.828 50.546) (width 0.3) (layer F.Cu) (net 5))
 (segment (start 133.096 52.672) (end 133.096 50.814) (width 0.3) (layer F.Cu) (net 5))
 (segment (start 122.061 49.372) (end 122.061 48.26) (width 0.3) (layer F.Cu) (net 5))
 (segment (start 122.03 49.403) (end 122.061 49.372) (width 0.3) (layer F.Cu) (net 5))
 (segment (start 132.828 50.546) (end 132.828 48.26) (width 0.3) (layer F.Cu) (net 5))
 (segment (start 128.651 54.356) (end 129.286 53.721) (width 0.3) (layer F.Cu) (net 5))
 (segment (start 127.494 54.356) (end 128.651 54.356) (width 0.3) (layer F.Cu) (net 5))
 (segment (start 129.286 52.672) (end 129.286 53.721) (width 0.3) (layer F.Cu) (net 5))
 (segment (start 129.286 53.721) (end 129.286 54.229) (width 0.3) (layer F.Cu) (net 5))
 (via (at 125.42062 47.04538) (size 0.7) (drill 0.4) (layers F.Cu B.Cu) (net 5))
 (segment (start 126.633 47.498) (end 125.87324 47.498) (width 0.3) (layer F.Cu) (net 5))
 (segment (start 125.87324 47.498) (end 125.42062 47.04538) (width 0.3) (layer F.Cu) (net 5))
 (segment (start 125.42062 47.04538) (end 125.42062 48.96662) (width 0.3) (layer B.Cu) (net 5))
 (via (at 125.476 49.022) (size 0.7) (drill 0.4) (layers F.Cu B.Cu) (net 5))
 (segment (start 125.42062 48.96662) (end 125.476 49.022) (width 0.3) (layer B.Cu) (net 5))
 (segment (start 125.476 50.278) (end 125.744 50.546) (width 0.3) (layer F.Cu) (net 5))
 (segment (start 125.476 49.022) (end 125.476 50.278) (width 0.3) (layer F.Cu) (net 5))
 (segment (start 130.578928 46.854072) (end 131.078 46.355) (width 0.2) (layer F.Cu) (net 12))
 (segment (start 129.921 47.512) (end 130.578928 46.854072) (width 0.2) (layer F.Cu) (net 12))
 (segment (start 129.921 51.181) (end 129.921 47.512) (width 0.2) (layer F.Cu) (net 12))
 (segment (start 130.556 52.672) (end 130.556 51.816) (width 0.2) (layer F.Cu) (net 12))
 (segment (start 130.556 51.816) (end 129.921 51.181) (width 0.2) (layer F.Cu) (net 12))
 (segment (start 131.078 44.845) (end 129.921 43.688) (width 0.2) (layer F.Cu) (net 12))
 (segment (start 131.078 46.355) (end 131.078 44.845) (width 0.2) (layer F.Cu) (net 12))
 (segment (start 129.935 47.498) (end 131.078 46.355) (width 0.2) (layer F.Cu) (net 12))
 (segment (start 128.383 47.498) (end 129.935 47.498) (width 0.2) (layer F.Cu) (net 12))
 (segment (start 122.061 46.51) (end 122.061 46.355) (width 0.2) (layer F.Cu) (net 17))
 (segment (start 123.811 48.26) (end 122.061 46.51) (width 0.2) (layer F.Cu) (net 17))
 (segment (start 132.828 46.51) (end 132.828 46.355) (width 0.2) (layer F.Cu) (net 16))
 (segment (start 131.078 48.26) (end 132.828 46.51) (width 0.2) (layer F.Cu) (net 16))
 (segment (start 125.716 56.035) (end 125.744 56.007) (width 0.2) (layer F.Cu) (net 15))
 (segment (start 125.716 57.658) (end 125.716 56.035) (width 0.2) (layer F.Cu) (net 15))
 (segment (start 128.173 59.778) (end 128.388 59.563) (width 0.3) (layer F.Cu) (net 4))
 (segment (start 128.173 60.753) (end 128.173 59.778) (width 0.3) (layer F.Cu) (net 4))
 (segment (start 131.318 59.563) (end 131.826 59.055) (width 0.3) (layer F.Cu) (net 4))
 (segment (start 128.388 59.563) (end 131.318 59.563) (width 0.3) (layer F.Cu) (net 4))
 (segment (start 131.826 59.055) (end 131.826 58.072) (width 0.3) (layer F.Cu) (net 4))
 (segment (start 124.46 55.118) (end 125.222 54.356) (width 0.3) (layer F.Cu) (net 4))
 (segment (start 123.966 57.658) (end 124.46 57.164) (width 0.3) (layer F.Cu) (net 4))
 (segment (start 125.222 54.356) (end 125.744 54.356) (width 0.3) (layer F.Cu) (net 4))
 (segment (start 124.46 57.164) (end 124.46 55.118) (width 0.3) (layer F.Cu) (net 4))
 (segment (start 128.230999 41.997999) (end 127.381 41.148) (width 0.3) (layer B.Cu) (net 4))
 (segment (start 128.651 42.418) (end 128.230999 41.997999) (width 0.3) (layer B.Cu) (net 4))
 (segment (start 132.461 43.688) (end 131.191 42.418) (width 0.3) (layer B.Cu) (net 4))
 (segment (start 131.191 42.418) (end 128.651 42.418) (width 0.3) (layer B.Cu) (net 4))
 (segment (start 124.371 50.951) (end 125.744 52.324) (width 0.3) (layer F.Cu) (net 4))
 (segment (start 123.632 50.951) (end 124.371 50.951) (width 0.3) (layer F.Cu) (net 4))
 (segment (start 125.744 52.296) (end 127.494 50.546) (width 0.3) (layer F.Cu) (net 4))
 (segment (start 125.744 52.324) (end 125.744 52.296) (width 0.3) (layer F.Cu) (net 4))
 (via (at 123.698 52.705) (size 0.7) (drill 0.4) (layers F.Cu B.Cu) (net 4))
 (segment (start 123.632 50.951) (end 123.632 52.639) (width 0.3) (layer F.Cu) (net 4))
 (segment (start 123.632 52.639) (end 123.698 52.705) (width 0.3) (layer F.Cu) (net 4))
 (via (at 131.826 49.403) (size 0.7) (drill 0.4) (layers F.Cu B.Cu) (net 4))
 (segment (start 131.078 50.546) (end 131.078 50.151) (width 0.3) (layer F.Cu) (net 4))
 (segment (start 131.078 50.151) (end 131.826 49.403) (width 0.3) (layer F.Cu) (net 4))
 (via (at 123.571 56.134) (size 0.7) (drill 0.4) (layers F.Cu B.Cu) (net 4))
 (segment (start 124.46 55.118) (end 124.46 55.245) (width 0.3) (layer F.Cu) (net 4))
 (segment (start 124.46 55.245) (end 123.571 56.134) (width 0.3) (layer F.Cu) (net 4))
 (via (at 132.334 60.706) (size 0.7) (drill 0.4) (layers F.Cu B.Cu) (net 4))
 (segment (start 131.826 58.072) (end 131.826 60.198) (width 0.3) (layer F.Cu) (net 4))
 (segment (start 131.826 60.198) (end 132.334 60.706) (width 0.3) (layer F.Cu) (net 4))
 (segment (start 128.076 60.85) (end 128.076 62.357) (width 0.3) (layer F.Cu) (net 4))
 (segment (start 128.173 60.753) (end 128.076 60.85) (width 0.3) (layer F.Cu) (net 4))
 (segment (start 127.426 63.007) (end 128.076 62.357) (width 0.3) (layer F.Cu) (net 4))
 (segment (start 127.426 63.357) (end 127.426 63.007) (width 0.3) (layer F.Cu) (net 4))
 (segment (start 130.131 62.357) (end 130.351 62.577) (width 0.3) (layer F.Cu) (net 4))
 (segment (start 128.076 62.357) (end 130.131 62.357) (width 0.3) (layer F.Cu) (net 4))
 (segment (start 126.873 60.753) (end 126.776 60.85) (width 0.2) (layer F.Cu) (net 3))
 (segment (start 126.873 59.878) (end 126.873 60.753) (width 0.2) (layer F.Cu) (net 3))
 (segment (start 126.776 60.85) (end 126.776 62.357) (width 0.2) (layer F.Cu) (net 3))
 (segment (start 129.286 58.072) (end 128.679 58.072) (width 0.2) (layer F.Cu) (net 3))
 (segment (start 128.679 58.072) (end 126.873 59.878) (width 0.2) (layer F.Cu) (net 3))
 (segment (start 130.556 57.023) (end 130.556 58.072) (width 0.2) (layer F.Cu) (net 2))
 (segment (start 130.175 56.642) (end 130.556 57.023) (width 0.2) (layer F.Cu) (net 2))
 (segment (start 128.778 56.642) (end 130.175 56.642) (width 0.2) (layer F.Cu) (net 2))
 (segment (start 126.223 60.753) (end 126.223 59.197) (width 0.2) (layer F.Cu) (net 2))
 (segment (start 126.223 59.197) (end 128.778 56.642) (width 0.2) (layer F.Cu) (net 2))
 (via (at 126.126 61.468) (size 0.6) (drill 0.3) (layers F.Cu B.Cu) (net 2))
 (segment (start 126.223 60.753) (end 126.223 61.371) (width 0.2) (layer F.Cu) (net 2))
 (segment (start 126.223 61.371) (end 126.126 61.468) (width 0.2) (layer F.Cu) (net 2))
 (segment (start 126.126 61.468) (end 125.095 61.468) (width 0.2) (layer B.Cu) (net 2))
 (segment (start 125.095 61.468) (end 124.714 61.849) (width 0.2) (layer B.Cu) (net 2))
 (segment (start 124.714 61.849) (end 124.714 63.246) (width 0.2) (layer B.Cu) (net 2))
 (segment (start 124.825 63.357) (end 126.126 63.357) (width 0.2) (layer B.Cu) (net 2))
 (segment (start 124.714 63.246) (end 124.825 63.357) (width 0.2) (layer B.Cu) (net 2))
 (via (at 131.699 54.356) (size 0.6) (drill 0.3) (layers F.Cu B.Cu) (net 13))
 (segment (start 131.826 52.672) (end 131.826 54.229) (width 0.2) (layer F.Cu) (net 13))
 (segment (start 131.826 54.229) (end 131.699 54.356) (width 0.2) (layer F.Cu) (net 13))
 (via (at 128.92012 49.13388) (size 0.6) (drill 0.3) (layers F.Cu B.Cu) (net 13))
 (segment (start 131.699 54.356) (end 128.92012 51.57712) (width 0.2) (layer B.Cu) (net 13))
 (segment (start 128.92012 51.57712) (end 128.92012 49.13388) (width 0.2) (layer B.Cu) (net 13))
 (segment (start 124.310072 46.854072) (end 123.811 46.355) (width 0.2) (layer F.Cu) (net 13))
 (segment (start 126.289881 48.833881) (end 124.310072 46.854072) (width 0.2) (layer F.Cu) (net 13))
 (segment (start 128.620121 48.833881) (end 126.289881 48.833881) (width 0.2) (layer F.Cu) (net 13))
 (segment (start 128.92012 49.13388) (end 128.620121 48.833881) (width 0.2) (layer F.Cu) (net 13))
 (segment (start 129.071001 41.997999) (end 129.921 41.148) (width 0.2) (layer F.Cu) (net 13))
 (segment (start 128.651 42.418) (end 129.071001 41.997999) (width 0.2) (layer F.Cu) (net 13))
 (segment (start 128.651 44.45) (end 128.651 42.418) (width 0.2) (layer F.Cu) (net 13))
 (segment (start 123.811 46.355) (end 126.746 46.355) (width 0.2) (layer F.Cu) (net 13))
 (segment (start 126.746 46.355) (end 128.651 44.45) (width 0.2) (layer F.Cu) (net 13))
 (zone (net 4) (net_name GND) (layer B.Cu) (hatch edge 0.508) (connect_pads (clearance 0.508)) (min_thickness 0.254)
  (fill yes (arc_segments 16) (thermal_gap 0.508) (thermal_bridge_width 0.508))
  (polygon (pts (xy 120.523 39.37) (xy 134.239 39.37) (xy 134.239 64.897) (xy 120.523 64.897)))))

